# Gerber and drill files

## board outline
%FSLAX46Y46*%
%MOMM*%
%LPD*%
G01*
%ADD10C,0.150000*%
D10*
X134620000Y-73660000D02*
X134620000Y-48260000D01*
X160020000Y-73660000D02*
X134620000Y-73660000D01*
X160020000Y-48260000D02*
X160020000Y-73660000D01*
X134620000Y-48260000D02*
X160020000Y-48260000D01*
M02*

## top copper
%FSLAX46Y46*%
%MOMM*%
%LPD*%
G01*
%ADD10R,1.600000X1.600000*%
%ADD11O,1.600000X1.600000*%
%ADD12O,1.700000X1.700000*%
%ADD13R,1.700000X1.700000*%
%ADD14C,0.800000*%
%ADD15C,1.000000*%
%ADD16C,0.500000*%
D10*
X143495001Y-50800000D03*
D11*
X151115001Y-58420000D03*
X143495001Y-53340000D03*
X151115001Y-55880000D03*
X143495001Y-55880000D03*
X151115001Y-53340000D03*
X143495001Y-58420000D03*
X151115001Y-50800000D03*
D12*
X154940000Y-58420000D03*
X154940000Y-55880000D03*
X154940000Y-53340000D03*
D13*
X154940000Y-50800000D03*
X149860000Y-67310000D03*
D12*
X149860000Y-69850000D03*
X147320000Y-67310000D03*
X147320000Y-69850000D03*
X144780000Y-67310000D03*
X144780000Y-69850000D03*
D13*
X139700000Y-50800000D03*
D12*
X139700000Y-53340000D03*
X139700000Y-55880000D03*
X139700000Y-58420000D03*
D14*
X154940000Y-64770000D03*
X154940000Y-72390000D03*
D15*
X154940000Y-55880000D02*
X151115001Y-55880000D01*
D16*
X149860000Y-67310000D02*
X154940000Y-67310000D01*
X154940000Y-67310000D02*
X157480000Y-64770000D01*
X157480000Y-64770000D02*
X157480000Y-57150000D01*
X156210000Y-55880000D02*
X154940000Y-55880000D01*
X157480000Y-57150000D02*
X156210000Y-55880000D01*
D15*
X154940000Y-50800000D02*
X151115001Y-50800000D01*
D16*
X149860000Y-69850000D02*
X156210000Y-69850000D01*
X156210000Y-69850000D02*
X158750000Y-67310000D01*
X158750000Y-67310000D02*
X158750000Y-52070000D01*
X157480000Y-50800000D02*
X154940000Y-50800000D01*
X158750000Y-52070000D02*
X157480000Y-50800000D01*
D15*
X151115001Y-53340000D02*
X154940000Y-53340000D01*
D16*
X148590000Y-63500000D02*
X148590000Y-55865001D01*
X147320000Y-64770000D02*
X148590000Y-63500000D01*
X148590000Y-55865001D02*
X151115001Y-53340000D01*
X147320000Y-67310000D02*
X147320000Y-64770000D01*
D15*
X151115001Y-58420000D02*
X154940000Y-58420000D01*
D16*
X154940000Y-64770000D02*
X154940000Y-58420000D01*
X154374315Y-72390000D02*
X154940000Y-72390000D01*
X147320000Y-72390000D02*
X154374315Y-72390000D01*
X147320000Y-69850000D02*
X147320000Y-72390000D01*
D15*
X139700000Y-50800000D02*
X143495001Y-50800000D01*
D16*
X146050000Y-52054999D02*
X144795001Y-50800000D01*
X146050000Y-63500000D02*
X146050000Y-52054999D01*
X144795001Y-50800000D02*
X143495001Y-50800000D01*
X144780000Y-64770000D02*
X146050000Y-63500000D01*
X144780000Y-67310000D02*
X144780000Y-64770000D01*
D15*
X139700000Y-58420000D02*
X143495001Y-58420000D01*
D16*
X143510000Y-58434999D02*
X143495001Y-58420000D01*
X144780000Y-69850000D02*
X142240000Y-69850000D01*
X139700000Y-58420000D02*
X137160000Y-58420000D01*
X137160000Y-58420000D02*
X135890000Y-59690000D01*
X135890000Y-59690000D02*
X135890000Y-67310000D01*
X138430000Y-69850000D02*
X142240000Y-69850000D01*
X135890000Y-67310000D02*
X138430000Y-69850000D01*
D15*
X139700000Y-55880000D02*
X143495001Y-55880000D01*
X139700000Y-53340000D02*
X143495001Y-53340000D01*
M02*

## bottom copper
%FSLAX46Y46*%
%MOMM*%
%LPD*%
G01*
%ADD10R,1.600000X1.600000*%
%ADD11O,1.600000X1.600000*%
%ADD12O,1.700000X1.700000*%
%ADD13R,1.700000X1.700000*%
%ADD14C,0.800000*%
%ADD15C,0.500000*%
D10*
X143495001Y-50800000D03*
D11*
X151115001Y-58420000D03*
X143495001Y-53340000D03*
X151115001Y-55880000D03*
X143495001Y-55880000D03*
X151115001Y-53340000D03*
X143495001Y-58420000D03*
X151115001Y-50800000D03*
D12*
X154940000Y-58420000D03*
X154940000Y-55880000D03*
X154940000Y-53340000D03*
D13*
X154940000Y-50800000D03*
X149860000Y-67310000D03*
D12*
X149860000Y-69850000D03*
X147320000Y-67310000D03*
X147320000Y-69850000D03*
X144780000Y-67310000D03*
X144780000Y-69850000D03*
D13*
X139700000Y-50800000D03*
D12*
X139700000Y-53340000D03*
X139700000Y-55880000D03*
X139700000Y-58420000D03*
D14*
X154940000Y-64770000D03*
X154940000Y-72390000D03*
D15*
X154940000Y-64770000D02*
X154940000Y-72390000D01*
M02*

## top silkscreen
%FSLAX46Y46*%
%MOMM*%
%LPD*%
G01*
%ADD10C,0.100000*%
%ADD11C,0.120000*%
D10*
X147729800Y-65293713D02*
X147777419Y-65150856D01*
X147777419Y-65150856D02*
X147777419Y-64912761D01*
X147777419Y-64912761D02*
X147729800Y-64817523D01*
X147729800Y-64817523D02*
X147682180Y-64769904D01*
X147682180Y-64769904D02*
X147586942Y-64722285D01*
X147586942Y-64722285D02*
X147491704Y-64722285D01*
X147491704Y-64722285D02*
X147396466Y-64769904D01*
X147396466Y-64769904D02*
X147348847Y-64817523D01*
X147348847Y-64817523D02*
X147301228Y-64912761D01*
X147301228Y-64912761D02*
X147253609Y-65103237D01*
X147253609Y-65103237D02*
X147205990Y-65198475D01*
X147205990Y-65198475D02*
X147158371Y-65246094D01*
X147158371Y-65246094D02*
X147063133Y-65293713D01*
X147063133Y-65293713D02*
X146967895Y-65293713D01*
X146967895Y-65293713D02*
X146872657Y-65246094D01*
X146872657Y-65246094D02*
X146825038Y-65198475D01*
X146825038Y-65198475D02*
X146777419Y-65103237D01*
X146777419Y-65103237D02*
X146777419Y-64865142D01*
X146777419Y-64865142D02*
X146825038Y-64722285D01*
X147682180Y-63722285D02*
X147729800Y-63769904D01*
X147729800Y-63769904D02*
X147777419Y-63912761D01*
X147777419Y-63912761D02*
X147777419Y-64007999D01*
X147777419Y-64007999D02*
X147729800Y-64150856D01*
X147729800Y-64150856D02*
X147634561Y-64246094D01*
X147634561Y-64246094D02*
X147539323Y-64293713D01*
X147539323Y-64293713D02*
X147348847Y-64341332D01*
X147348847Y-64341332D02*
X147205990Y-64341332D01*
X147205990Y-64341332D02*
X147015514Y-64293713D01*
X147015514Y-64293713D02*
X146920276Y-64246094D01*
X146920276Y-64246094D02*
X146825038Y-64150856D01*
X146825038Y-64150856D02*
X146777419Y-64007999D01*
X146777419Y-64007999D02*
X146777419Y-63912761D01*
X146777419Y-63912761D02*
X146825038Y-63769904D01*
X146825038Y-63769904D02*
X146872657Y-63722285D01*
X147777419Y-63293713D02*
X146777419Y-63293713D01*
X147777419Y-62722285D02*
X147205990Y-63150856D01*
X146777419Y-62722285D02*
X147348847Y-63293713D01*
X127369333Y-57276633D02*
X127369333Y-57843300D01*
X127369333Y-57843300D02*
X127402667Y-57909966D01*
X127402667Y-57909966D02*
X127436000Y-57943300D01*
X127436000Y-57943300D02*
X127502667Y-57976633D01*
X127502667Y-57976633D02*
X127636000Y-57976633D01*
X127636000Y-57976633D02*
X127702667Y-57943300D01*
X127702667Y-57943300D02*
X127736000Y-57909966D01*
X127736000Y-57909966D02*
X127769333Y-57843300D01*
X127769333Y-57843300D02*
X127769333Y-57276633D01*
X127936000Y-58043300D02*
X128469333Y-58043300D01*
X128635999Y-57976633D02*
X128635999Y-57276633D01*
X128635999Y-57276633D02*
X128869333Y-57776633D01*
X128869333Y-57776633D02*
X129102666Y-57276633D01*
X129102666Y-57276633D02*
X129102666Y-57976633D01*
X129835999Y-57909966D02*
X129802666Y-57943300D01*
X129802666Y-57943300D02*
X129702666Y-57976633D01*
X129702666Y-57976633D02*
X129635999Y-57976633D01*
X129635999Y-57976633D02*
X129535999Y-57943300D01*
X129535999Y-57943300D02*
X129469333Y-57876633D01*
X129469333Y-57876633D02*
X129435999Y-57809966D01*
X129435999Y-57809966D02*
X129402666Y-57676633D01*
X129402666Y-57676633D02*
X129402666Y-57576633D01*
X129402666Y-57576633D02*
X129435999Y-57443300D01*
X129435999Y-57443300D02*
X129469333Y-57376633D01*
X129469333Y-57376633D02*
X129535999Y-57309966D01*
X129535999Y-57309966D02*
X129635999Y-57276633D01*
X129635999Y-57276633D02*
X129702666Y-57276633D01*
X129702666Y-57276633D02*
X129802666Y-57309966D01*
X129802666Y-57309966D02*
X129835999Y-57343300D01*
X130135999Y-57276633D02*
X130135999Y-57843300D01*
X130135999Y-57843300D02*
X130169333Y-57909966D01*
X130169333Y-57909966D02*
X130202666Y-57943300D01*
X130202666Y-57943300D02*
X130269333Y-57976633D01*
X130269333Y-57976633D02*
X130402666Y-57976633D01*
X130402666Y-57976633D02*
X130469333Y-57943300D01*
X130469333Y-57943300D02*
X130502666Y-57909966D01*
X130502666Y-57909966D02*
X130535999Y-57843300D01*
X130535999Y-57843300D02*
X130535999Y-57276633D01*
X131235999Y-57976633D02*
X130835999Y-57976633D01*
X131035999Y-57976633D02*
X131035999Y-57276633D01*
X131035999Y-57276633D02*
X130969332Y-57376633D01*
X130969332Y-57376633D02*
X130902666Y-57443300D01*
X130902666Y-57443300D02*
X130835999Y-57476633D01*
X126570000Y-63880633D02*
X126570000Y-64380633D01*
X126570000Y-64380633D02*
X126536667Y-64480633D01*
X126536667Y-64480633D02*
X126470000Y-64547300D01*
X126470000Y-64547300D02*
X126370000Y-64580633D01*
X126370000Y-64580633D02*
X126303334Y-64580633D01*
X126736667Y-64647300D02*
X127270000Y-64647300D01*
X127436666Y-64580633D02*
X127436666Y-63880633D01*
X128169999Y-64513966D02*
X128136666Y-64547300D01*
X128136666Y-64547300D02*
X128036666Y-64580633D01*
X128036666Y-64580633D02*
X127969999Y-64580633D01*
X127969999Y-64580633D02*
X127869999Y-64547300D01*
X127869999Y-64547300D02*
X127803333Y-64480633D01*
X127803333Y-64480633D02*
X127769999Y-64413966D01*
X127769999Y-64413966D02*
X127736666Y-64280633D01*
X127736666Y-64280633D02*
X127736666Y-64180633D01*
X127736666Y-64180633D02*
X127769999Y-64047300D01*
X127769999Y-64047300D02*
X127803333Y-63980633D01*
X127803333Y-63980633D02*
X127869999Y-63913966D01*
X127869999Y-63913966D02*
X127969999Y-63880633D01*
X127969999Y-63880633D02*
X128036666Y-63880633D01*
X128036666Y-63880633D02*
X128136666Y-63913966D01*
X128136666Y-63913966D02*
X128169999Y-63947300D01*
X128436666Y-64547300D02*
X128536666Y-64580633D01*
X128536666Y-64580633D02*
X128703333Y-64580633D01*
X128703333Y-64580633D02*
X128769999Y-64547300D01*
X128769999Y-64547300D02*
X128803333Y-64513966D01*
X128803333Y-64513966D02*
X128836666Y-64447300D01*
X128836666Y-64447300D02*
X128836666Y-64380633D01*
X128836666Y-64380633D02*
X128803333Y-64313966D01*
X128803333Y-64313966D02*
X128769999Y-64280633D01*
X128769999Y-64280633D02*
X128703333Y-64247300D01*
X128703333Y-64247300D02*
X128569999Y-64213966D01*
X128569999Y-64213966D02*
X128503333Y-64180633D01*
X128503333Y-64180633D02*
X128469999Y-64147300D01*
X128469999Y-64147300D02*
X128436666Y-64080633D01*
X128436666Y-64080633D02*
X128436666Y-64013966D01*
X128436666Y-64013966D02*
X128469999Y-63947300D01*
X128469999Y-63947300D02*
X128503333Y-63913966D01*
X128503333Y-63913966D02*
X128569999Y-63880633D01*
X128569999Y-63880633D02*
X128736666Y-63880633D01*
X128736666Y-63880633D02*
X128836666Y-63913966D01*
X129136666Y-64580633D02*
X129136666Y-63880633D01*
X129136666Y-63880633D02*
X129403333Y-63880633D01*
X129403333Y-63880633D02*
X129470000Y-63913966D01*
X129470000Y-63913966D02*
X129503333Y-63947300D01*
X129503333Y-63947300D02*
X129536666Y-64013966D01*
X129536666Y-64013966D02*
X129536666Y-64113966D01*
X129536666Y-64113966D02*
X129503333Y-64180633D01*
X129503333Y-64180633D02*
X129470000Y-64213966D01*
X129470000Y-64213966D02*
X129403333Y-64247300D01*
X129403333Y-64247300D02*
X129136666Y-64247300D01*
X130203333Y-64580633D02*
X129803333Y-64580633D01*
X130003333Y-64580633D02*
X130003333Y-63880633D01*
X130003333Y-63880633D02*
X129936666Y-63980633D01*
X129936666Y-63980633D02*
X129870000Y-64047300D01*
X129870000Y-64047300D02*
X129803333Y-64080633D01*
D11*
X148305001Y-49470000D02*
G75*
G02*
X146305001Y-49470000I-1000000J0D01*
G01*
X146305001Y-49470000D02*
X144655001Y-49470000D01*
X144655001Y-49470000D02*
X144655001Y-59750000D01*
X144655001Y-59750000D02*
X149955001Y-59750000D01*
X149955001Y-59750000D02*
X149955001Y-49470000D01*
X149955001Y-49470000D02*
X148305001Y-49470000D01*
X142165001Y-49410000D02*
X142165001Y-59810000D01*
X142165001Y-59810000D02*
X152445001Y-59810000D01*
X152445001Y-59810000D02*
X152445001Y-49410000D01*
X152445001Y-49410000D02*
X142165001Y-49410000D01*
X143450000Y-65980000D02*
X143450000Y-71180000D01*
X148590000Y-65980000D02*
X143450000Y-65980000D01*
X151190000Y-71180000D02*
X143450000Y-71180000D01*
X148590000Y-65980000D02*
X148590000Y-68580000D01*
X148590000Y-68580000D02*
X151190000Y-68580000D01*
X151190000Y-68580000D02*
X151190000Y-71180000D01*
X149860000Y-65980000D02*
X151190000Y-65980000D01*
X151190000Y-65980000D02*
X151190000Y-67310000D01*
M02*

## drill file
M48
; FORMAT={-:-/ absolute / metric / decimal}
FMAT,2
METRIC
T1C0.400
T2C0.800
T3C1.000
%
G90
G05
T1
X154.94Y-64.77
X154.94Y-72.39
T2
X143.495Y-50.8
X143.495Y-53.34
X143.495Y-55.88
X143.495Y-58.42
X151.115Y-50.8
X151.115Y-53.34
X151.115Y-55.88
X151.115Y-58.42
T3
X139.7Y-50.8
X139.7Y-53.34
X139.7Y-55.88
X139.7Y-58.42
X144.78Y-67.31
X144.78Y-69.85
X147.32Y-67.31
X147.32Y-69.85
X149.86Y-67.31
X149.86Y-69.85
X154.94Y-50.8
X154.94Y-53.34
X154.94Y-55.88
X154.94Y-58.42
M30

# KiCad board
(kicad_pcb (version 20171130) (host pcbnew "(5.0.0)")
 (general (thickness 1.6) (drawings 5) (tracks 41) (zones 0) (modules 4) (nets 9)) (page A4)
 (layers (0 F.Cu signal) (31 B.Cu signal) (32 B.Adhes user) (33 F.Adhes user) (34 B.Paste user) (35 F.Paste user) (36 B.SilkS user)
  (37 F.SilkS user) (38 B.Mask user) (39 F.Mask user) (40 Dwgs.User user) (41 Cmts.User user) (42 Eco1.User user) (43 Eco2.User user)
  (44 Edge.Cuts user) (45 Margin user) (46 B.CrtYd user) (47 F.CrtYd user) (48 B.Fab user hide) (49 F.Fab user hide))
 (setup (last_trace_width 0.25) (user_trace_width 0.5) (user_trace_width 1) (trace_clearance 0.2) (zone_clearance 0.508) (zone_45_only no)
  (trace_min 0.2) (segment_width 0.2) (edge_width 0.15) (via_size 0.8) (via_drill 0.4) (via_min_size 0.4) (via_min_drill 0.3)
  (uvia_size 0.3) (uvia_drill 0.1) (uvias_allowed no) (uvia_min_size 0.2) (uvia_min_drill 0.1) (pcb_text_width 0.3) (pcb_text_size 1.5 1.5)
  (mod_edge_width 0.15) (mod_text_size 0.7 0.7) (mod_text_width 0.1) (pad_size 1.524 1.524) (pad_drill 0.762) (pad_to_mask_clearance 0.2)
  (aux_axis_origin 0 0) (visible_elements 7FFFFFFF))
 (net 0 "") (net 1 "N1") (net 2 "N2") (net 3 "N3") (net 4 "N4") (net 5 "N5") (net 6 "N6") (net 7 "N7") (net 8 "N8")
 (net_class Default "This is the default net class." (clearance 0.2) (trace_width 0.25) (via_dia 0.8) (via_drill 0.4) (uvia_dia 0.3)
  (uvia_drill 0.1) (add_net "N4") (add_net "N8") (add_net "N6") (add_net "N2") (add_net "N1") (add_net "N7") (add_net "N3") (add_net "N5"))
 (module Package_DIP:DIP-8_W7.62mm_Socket (layer F.Cu) (at 143.495001 50.8)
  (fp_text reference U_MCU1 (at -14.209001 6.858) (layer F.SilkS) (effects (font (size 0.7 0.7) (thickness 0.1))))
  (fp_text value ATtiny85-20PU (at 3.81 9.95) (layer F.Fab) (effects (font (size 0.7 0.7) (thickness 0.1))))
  (fp_arc (start 3.81 -1.33) (end 2.81 -1.33) (angle -180) (layer F.SilkS) (width 0.12))
  (fp_line (start 2.81 -1.33) (end 1.16 -1.33) (layer F.SilkS) (width 0.12))
  (fp_line (start 1.16 -1.33) (end 1.16 8.95) (layer F.SilkS) (width 0.12))
  (fp_line (start 1.16 8.95) (end 6.46 8.95) (layer F.SilkS) (width 0.12))
  (fp_line (start 6.46 8.95) (end 6.46 -1.33) (layer F.SilkS) (width 0.12))
  (fp_line (start 6.46 -1.33) (end 4.81 -1.33) (layer F.SilkS) (width 0.12))
  (fp_line (start -1.33 -1.39) (end -1.33 9.01) (layer F.SilkS) (width 0.12))
  (fp_line (start -1.33 9.01) (end 8.95 9.01) (layer F.SilkS) (width 0.12))
  (fp_line (start 8.95 9.01) (end 8.95 -1.39) (layer F.SilkS) (width 0.12))
  (fp_line (start 8.95 -1.39) (end -1.33 -1.39) (layer F.SilkS) (width 0.12))
  (pad 1 thru_hole rect (at 0 0) (size 1.6 1.6) (drill 0.8) (layers *.Cu *.Mask) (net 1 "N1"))
  (pad 5 thru_hole oval (at 7.62 7.62) (size 1.6 1.6) (drill 0.8) (layers *.Cu *.Mask) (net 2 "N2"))
  (pad 2 thru_hole oval (at 0 2.54) (size 1.6 1.6) (drill 0.8) (layers *.Cu *.Mask) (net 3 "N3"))
  (pad 6 thru_hole oval (at 7.62 5.08) (size 1.6 1.6) (drill 0.8) (layers *.Cu *.Mask) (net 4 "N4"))
  (pad 3 thru_hole oval (at 0 5.08) (size 1.6 1.6) (drill 0.8) (layers *.Cu *.Mask) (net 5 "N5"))
  (pad 7 thru_hole oval (at 7.62 2.54) (size 1.6 1.6) (drill 0.8) (layers *.Cu *.Mask) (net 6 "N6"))
  (pad 4 thru_hole oval (at 0 7.62) (size 1.6 1.6) (drill 0.8) (layers *.Cu *.Mask) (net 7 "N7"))
  (pad 8 thru_hole oval (at 7.62 0) (size 1.6 1.6) (drill 0.8) (layers *.Cu *.Mask) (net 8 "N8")))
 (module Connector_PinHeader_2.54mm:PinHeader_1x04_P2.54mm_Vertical (layer B.Cu) (at 154.94 50.8 180)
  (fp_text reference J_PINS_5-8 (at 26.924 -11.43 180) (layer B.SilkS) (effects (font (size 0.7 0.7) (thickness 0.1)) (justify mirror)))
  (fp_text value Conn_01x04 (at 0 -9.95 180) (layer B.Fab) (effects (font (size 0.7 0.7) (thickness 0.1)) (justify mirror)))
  (pad 4 thru_hole oval (at 0 -7.62 180) (size 1.7 1.7) (drill 1) (layers *.Cu *.Mask) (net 2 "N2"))
  (pad 3 thru_hole oval (at 0 -5.08 180) (size 1.7 1.7) (drill 1) (layers *.Cu *.Mask) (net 4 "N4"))
  (pad 2 thru_hole oval (at 0 -2.54 180) (size 1.7 1.7) (drill 1) (layers *.Cu *.Mask) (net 6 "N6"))
  (pad 1 thru_hole rect (at 0 0 180) (size 1.7 1.7) (drill 1) (layers *.Cu *.Mask) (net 8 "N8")))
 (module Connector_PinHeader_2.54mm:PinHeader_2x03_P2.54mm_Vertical (layer F.Cu) (at 149.86 67.31 270)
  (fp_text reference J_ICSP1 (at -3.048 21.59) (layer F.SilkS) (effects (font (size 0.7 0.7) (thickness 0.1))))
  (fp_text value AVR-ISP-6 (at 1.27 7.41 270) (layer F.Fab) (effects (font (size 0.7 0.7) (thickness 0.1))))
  (fp_line (start -1.33 6.41) (end 3.87 6.41) (layer F.SilkS) (width 0.12))
  (fp_line (start -1.33 1.27) (end -1.33 6.41) (layer F.SilkS) (width 0.12))
  (fp_line (start 3.87 -1.33) (end 3.87 6.41) (layer F.SilkS) (width 0.12))
  (fp_line (start -1.33 1.27) (end 1.27 1.27) (layer F.SilkS) (width 0.12))
  (fp_line (start 1.27 1.27) (end 1.27 -1.33) (layer F.SilkS) (width 0.12))
  (fp_line (start 1.27 -1.33) (end 3.87 -1.33) (layer F.SilkS) (width 0.12))
  (fp_line (start -1.33 0) (end -1.33 -1.33) (layer F.SilkS) (width 0.12))
  (fp_line (start -1.33 -1.33) (end 0 -1.33) (layer F.SilkS) (width 0.12))
  (pad 1 thru_hole rect (at 0 0 270) (size 1.7 1.7) (drill 1) (layers *.Cu *.Mask) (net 4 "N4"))
  (pad 2 thru_hole oval (at 2.54 0 270) (size 1.7 1.7) (drill 1) (layers *.Cu *.Mask) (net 8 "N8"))
  (pad 3 thru_hole oval (at 0 2.54 270) (size 1.7 1.7) (drill 1) (layers *.Cu *.Mask) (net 6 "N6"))
  (pad 4 thru_hole oval (at 2.54 2.54 270) (size 1.7 1.7) (drill 1) (layers *.Cu *.Mask) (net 2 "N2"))
  (pad 5 thru_hole oval (at 0 5.08 270) (size 1.7 1.7) (drill 1) (layers *.Cu *.Mask) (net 1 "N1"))
  (pad 6 thru_hole oval (at 2.54 5.08 270) (size 1.7 1.7) (drill 1) (layers *.Cu *.Mask) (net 7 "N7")))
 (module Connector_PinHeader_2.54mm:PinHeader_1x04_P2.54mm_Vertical (layer B.Cu) (at 139.7 50.8 180)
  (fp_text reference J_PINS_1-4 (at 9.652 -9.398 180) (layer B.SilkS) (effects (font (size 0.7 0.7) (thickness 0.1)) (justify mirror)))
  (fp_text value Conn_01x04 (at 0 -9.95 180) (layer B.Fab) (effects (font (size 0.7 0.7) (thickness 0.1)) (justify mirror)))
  (pad 1 thru_hole rect (at 0 0 180) (size 1.7 1.7) (drill 1) (layers *.Cu *.Mask) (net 1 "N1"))
  (pad 2 thru_hole oval (at 0 -2.54 180) (size 1.7 1.7) (drill 1) (layers *.Cu *.Mask) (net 3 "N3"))
  (pad 3 thru_hole oval (at 0 -5.08 180) (size 1.7 1.7) (drill 1) (layers *.Cu *.Mask) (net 5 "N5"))
  (pad 4 thru_hole oval (at 0 -7.62 180) (size 1.7 1.7) (drill 1) (layers *.Cu *.Mask) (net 7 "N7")))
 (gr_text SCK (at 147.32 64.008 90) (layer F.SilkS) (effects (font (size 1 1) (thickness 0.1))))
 (gr_line (start 134.62 73.66) (end 134.62 48.26) (layer Edge.Cuts) (width 0.15))
 (gr_line (start 160.02 73.66) (end 134.62 73.66) (layer Edge.Cuts) (width 0.15))
 (gr_line (start 160.02 48.26) (end 160.02 73.66) (layer Edge.Cuts) (width 0.15))
 (gr_line (start 134.62 48.26) (end 160.02 48.26) (layer Edge.Cuts) (width 0.15))
 (segment (start 154.94 55.88) (end 151.115001 55.88) (width 1) (layer F.Cu) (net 4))
 (segment (start 149.86 67.31) (end 154.94 67.31) (width 0.5) (layer F.Cu) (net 4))
 (segment (start 154.94 67.31) (end 157.48 64.77) (width 0.5) (layer F.Cu) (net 4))
 (segment (start 157.48 64.77) (end 157.48 57.15) (width 0.5) (layer F.Cu) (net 4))
 (segment (start 156.21 55.88) (end 154.94 55.88) (width 0.5) (layer F.Cu) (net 4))
 (segment (start 157.48 57.15) (end 156.21 55.88) (width 0.5) (layer F.Cu) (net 4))
 (segment (start 154.94 50.8) (end 151.115001 50.8) (width 1) (layer F.Cu) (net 8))
 (segment (start 149.86 69.85) (end 156.21 69.85) (width 0.5) (layer F.Cu) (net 8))
 (segment (start 156.21 69.85) (end 158.75 67.31) (width 0.5) (layer F.Cu) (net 8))
 (segment (start 158.75 67.31) (end 158.75 52.07) (width 0.5) (layer F.Cu) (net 8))
 (segment (start 157.48 50.8) (end 154.94 50.8) (width 0.5) (layer F.Cu) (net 8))
 (segment (start 158.75 52.07) (end 157.48 50.8) (width 0.5) (layer F.Cu) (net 8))
 (segment (start 151.115001 53.34) (end 154.94 53.34) (width 1) (layer F.Cu) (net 6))
 (segment (start 148.59 63.5) (end 148.59 55.865001) (width 0.5) (layer F.Cu) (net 6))
 (segment (start 147.32 64.77) (end 148.59 63.5) (width 0.5) (layer F.Cu) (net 6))
 (segment (start 148.59 55.865001) (end 151.115001 53.34) (width 0.5) (layer F.Cu) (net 6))
 (segment (start 147.32 67.31) (end 147.32 64.77) (width 0.5) (layer F.Cu) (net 6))
 (segment (start 151.115001 58.42) (end 154.94 58.42) (width 1) (layer F.Cu) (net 2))
 (via (at 154.94 64.77) (size 0.8) (drill 0.4) (layers F.Cu B.Cu) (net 2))
 (segment (start 154.94 64.77) (end 154.94 58.42) (width 0.5) (layer F.Cu) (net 2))
 (segment (start 154.94 64.77) (end 154.94 72.39) (width 0.5) (layer B.Cu) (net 2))
 (via (at 154.94 72.39) (size 0.8) (drill 0.4) (layers F.Cu B.Cu) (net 2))
 (segment (start 154.374315 72.39) (end 154.94 72.39) (width 0.5) (layer F.Cu) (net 2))
 (segment (start 147.32 72.39) (end 154.374315 72.39) (width 0.5) (layer F.Cu) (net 2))
 (segment (start 147.32 69.85) (end 147.32 72.39) (width 0.5) (layer F.Cu) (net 2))
 (segment (start 139.7 50.8) (end 143.495001 50.8) (width 1) (layer F.Cu) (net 1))
 (segment (start 146.05 52.054999) (end 144.795001 50.8) (width 0.5) (layer F.Cu) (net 1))
 (segment (start 146.05 63.5) (end 146.05 52.054999) (width 0.5) (layer F.Cu) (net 1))
 (segment (start 144.795001 50.8) (end 143.495001 50.8) (width 0.5) (layer F.Cu) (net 1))
 (segment (start 144.78 64.77) (end 146.05 63.5) (width 0.5) (layer F.Cu) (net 1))
 (segment (start 144.78 67.31) (end 144.78 64.77) (width 0.5) (layer F.Cu) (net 1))
 (segment (start 139.7 58.42) (end 143.495001 58.42) (width 1) (layer F.Cu) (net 7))
 (segment (start 143.51 58.434999) (end 143.495001 58.42) (width 0.5) (layer F.Cu) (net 7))
 (segment (start 144.78 69.85) (end 142.24 69.85) (width 0.5) (layer F.Cu) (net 7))
 (segment (start 139.7 58.42) (end 137.16 58.42) (width 0.5) (layer F.Cu) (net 7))
 (segment (start 137.16 58.42) (end 135.89 59.69) (width 0.5) (layer F.Cu) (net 7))
 (segment (start 135.89 59.69) (end 135.89 67.31) (width 0.5) (layer F.Cu) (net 7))
 (segment (start 138.43 69.85) (end 142.24 69.85) (width 0.5) (layer F.Cu) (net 7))
 (segment (start 135.89 67.31) (end 138.43 69.85) (width 0.5) (layer F.Cu) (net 7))
 (segment (start 139.7 55.88) (end 143.495001 55.88) (width 1) (layer F.Cu) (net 5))
 (segment (start 139.7 53.34) (end 143.495001 53.34) (width 1) (layer F.Cu) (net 3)))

